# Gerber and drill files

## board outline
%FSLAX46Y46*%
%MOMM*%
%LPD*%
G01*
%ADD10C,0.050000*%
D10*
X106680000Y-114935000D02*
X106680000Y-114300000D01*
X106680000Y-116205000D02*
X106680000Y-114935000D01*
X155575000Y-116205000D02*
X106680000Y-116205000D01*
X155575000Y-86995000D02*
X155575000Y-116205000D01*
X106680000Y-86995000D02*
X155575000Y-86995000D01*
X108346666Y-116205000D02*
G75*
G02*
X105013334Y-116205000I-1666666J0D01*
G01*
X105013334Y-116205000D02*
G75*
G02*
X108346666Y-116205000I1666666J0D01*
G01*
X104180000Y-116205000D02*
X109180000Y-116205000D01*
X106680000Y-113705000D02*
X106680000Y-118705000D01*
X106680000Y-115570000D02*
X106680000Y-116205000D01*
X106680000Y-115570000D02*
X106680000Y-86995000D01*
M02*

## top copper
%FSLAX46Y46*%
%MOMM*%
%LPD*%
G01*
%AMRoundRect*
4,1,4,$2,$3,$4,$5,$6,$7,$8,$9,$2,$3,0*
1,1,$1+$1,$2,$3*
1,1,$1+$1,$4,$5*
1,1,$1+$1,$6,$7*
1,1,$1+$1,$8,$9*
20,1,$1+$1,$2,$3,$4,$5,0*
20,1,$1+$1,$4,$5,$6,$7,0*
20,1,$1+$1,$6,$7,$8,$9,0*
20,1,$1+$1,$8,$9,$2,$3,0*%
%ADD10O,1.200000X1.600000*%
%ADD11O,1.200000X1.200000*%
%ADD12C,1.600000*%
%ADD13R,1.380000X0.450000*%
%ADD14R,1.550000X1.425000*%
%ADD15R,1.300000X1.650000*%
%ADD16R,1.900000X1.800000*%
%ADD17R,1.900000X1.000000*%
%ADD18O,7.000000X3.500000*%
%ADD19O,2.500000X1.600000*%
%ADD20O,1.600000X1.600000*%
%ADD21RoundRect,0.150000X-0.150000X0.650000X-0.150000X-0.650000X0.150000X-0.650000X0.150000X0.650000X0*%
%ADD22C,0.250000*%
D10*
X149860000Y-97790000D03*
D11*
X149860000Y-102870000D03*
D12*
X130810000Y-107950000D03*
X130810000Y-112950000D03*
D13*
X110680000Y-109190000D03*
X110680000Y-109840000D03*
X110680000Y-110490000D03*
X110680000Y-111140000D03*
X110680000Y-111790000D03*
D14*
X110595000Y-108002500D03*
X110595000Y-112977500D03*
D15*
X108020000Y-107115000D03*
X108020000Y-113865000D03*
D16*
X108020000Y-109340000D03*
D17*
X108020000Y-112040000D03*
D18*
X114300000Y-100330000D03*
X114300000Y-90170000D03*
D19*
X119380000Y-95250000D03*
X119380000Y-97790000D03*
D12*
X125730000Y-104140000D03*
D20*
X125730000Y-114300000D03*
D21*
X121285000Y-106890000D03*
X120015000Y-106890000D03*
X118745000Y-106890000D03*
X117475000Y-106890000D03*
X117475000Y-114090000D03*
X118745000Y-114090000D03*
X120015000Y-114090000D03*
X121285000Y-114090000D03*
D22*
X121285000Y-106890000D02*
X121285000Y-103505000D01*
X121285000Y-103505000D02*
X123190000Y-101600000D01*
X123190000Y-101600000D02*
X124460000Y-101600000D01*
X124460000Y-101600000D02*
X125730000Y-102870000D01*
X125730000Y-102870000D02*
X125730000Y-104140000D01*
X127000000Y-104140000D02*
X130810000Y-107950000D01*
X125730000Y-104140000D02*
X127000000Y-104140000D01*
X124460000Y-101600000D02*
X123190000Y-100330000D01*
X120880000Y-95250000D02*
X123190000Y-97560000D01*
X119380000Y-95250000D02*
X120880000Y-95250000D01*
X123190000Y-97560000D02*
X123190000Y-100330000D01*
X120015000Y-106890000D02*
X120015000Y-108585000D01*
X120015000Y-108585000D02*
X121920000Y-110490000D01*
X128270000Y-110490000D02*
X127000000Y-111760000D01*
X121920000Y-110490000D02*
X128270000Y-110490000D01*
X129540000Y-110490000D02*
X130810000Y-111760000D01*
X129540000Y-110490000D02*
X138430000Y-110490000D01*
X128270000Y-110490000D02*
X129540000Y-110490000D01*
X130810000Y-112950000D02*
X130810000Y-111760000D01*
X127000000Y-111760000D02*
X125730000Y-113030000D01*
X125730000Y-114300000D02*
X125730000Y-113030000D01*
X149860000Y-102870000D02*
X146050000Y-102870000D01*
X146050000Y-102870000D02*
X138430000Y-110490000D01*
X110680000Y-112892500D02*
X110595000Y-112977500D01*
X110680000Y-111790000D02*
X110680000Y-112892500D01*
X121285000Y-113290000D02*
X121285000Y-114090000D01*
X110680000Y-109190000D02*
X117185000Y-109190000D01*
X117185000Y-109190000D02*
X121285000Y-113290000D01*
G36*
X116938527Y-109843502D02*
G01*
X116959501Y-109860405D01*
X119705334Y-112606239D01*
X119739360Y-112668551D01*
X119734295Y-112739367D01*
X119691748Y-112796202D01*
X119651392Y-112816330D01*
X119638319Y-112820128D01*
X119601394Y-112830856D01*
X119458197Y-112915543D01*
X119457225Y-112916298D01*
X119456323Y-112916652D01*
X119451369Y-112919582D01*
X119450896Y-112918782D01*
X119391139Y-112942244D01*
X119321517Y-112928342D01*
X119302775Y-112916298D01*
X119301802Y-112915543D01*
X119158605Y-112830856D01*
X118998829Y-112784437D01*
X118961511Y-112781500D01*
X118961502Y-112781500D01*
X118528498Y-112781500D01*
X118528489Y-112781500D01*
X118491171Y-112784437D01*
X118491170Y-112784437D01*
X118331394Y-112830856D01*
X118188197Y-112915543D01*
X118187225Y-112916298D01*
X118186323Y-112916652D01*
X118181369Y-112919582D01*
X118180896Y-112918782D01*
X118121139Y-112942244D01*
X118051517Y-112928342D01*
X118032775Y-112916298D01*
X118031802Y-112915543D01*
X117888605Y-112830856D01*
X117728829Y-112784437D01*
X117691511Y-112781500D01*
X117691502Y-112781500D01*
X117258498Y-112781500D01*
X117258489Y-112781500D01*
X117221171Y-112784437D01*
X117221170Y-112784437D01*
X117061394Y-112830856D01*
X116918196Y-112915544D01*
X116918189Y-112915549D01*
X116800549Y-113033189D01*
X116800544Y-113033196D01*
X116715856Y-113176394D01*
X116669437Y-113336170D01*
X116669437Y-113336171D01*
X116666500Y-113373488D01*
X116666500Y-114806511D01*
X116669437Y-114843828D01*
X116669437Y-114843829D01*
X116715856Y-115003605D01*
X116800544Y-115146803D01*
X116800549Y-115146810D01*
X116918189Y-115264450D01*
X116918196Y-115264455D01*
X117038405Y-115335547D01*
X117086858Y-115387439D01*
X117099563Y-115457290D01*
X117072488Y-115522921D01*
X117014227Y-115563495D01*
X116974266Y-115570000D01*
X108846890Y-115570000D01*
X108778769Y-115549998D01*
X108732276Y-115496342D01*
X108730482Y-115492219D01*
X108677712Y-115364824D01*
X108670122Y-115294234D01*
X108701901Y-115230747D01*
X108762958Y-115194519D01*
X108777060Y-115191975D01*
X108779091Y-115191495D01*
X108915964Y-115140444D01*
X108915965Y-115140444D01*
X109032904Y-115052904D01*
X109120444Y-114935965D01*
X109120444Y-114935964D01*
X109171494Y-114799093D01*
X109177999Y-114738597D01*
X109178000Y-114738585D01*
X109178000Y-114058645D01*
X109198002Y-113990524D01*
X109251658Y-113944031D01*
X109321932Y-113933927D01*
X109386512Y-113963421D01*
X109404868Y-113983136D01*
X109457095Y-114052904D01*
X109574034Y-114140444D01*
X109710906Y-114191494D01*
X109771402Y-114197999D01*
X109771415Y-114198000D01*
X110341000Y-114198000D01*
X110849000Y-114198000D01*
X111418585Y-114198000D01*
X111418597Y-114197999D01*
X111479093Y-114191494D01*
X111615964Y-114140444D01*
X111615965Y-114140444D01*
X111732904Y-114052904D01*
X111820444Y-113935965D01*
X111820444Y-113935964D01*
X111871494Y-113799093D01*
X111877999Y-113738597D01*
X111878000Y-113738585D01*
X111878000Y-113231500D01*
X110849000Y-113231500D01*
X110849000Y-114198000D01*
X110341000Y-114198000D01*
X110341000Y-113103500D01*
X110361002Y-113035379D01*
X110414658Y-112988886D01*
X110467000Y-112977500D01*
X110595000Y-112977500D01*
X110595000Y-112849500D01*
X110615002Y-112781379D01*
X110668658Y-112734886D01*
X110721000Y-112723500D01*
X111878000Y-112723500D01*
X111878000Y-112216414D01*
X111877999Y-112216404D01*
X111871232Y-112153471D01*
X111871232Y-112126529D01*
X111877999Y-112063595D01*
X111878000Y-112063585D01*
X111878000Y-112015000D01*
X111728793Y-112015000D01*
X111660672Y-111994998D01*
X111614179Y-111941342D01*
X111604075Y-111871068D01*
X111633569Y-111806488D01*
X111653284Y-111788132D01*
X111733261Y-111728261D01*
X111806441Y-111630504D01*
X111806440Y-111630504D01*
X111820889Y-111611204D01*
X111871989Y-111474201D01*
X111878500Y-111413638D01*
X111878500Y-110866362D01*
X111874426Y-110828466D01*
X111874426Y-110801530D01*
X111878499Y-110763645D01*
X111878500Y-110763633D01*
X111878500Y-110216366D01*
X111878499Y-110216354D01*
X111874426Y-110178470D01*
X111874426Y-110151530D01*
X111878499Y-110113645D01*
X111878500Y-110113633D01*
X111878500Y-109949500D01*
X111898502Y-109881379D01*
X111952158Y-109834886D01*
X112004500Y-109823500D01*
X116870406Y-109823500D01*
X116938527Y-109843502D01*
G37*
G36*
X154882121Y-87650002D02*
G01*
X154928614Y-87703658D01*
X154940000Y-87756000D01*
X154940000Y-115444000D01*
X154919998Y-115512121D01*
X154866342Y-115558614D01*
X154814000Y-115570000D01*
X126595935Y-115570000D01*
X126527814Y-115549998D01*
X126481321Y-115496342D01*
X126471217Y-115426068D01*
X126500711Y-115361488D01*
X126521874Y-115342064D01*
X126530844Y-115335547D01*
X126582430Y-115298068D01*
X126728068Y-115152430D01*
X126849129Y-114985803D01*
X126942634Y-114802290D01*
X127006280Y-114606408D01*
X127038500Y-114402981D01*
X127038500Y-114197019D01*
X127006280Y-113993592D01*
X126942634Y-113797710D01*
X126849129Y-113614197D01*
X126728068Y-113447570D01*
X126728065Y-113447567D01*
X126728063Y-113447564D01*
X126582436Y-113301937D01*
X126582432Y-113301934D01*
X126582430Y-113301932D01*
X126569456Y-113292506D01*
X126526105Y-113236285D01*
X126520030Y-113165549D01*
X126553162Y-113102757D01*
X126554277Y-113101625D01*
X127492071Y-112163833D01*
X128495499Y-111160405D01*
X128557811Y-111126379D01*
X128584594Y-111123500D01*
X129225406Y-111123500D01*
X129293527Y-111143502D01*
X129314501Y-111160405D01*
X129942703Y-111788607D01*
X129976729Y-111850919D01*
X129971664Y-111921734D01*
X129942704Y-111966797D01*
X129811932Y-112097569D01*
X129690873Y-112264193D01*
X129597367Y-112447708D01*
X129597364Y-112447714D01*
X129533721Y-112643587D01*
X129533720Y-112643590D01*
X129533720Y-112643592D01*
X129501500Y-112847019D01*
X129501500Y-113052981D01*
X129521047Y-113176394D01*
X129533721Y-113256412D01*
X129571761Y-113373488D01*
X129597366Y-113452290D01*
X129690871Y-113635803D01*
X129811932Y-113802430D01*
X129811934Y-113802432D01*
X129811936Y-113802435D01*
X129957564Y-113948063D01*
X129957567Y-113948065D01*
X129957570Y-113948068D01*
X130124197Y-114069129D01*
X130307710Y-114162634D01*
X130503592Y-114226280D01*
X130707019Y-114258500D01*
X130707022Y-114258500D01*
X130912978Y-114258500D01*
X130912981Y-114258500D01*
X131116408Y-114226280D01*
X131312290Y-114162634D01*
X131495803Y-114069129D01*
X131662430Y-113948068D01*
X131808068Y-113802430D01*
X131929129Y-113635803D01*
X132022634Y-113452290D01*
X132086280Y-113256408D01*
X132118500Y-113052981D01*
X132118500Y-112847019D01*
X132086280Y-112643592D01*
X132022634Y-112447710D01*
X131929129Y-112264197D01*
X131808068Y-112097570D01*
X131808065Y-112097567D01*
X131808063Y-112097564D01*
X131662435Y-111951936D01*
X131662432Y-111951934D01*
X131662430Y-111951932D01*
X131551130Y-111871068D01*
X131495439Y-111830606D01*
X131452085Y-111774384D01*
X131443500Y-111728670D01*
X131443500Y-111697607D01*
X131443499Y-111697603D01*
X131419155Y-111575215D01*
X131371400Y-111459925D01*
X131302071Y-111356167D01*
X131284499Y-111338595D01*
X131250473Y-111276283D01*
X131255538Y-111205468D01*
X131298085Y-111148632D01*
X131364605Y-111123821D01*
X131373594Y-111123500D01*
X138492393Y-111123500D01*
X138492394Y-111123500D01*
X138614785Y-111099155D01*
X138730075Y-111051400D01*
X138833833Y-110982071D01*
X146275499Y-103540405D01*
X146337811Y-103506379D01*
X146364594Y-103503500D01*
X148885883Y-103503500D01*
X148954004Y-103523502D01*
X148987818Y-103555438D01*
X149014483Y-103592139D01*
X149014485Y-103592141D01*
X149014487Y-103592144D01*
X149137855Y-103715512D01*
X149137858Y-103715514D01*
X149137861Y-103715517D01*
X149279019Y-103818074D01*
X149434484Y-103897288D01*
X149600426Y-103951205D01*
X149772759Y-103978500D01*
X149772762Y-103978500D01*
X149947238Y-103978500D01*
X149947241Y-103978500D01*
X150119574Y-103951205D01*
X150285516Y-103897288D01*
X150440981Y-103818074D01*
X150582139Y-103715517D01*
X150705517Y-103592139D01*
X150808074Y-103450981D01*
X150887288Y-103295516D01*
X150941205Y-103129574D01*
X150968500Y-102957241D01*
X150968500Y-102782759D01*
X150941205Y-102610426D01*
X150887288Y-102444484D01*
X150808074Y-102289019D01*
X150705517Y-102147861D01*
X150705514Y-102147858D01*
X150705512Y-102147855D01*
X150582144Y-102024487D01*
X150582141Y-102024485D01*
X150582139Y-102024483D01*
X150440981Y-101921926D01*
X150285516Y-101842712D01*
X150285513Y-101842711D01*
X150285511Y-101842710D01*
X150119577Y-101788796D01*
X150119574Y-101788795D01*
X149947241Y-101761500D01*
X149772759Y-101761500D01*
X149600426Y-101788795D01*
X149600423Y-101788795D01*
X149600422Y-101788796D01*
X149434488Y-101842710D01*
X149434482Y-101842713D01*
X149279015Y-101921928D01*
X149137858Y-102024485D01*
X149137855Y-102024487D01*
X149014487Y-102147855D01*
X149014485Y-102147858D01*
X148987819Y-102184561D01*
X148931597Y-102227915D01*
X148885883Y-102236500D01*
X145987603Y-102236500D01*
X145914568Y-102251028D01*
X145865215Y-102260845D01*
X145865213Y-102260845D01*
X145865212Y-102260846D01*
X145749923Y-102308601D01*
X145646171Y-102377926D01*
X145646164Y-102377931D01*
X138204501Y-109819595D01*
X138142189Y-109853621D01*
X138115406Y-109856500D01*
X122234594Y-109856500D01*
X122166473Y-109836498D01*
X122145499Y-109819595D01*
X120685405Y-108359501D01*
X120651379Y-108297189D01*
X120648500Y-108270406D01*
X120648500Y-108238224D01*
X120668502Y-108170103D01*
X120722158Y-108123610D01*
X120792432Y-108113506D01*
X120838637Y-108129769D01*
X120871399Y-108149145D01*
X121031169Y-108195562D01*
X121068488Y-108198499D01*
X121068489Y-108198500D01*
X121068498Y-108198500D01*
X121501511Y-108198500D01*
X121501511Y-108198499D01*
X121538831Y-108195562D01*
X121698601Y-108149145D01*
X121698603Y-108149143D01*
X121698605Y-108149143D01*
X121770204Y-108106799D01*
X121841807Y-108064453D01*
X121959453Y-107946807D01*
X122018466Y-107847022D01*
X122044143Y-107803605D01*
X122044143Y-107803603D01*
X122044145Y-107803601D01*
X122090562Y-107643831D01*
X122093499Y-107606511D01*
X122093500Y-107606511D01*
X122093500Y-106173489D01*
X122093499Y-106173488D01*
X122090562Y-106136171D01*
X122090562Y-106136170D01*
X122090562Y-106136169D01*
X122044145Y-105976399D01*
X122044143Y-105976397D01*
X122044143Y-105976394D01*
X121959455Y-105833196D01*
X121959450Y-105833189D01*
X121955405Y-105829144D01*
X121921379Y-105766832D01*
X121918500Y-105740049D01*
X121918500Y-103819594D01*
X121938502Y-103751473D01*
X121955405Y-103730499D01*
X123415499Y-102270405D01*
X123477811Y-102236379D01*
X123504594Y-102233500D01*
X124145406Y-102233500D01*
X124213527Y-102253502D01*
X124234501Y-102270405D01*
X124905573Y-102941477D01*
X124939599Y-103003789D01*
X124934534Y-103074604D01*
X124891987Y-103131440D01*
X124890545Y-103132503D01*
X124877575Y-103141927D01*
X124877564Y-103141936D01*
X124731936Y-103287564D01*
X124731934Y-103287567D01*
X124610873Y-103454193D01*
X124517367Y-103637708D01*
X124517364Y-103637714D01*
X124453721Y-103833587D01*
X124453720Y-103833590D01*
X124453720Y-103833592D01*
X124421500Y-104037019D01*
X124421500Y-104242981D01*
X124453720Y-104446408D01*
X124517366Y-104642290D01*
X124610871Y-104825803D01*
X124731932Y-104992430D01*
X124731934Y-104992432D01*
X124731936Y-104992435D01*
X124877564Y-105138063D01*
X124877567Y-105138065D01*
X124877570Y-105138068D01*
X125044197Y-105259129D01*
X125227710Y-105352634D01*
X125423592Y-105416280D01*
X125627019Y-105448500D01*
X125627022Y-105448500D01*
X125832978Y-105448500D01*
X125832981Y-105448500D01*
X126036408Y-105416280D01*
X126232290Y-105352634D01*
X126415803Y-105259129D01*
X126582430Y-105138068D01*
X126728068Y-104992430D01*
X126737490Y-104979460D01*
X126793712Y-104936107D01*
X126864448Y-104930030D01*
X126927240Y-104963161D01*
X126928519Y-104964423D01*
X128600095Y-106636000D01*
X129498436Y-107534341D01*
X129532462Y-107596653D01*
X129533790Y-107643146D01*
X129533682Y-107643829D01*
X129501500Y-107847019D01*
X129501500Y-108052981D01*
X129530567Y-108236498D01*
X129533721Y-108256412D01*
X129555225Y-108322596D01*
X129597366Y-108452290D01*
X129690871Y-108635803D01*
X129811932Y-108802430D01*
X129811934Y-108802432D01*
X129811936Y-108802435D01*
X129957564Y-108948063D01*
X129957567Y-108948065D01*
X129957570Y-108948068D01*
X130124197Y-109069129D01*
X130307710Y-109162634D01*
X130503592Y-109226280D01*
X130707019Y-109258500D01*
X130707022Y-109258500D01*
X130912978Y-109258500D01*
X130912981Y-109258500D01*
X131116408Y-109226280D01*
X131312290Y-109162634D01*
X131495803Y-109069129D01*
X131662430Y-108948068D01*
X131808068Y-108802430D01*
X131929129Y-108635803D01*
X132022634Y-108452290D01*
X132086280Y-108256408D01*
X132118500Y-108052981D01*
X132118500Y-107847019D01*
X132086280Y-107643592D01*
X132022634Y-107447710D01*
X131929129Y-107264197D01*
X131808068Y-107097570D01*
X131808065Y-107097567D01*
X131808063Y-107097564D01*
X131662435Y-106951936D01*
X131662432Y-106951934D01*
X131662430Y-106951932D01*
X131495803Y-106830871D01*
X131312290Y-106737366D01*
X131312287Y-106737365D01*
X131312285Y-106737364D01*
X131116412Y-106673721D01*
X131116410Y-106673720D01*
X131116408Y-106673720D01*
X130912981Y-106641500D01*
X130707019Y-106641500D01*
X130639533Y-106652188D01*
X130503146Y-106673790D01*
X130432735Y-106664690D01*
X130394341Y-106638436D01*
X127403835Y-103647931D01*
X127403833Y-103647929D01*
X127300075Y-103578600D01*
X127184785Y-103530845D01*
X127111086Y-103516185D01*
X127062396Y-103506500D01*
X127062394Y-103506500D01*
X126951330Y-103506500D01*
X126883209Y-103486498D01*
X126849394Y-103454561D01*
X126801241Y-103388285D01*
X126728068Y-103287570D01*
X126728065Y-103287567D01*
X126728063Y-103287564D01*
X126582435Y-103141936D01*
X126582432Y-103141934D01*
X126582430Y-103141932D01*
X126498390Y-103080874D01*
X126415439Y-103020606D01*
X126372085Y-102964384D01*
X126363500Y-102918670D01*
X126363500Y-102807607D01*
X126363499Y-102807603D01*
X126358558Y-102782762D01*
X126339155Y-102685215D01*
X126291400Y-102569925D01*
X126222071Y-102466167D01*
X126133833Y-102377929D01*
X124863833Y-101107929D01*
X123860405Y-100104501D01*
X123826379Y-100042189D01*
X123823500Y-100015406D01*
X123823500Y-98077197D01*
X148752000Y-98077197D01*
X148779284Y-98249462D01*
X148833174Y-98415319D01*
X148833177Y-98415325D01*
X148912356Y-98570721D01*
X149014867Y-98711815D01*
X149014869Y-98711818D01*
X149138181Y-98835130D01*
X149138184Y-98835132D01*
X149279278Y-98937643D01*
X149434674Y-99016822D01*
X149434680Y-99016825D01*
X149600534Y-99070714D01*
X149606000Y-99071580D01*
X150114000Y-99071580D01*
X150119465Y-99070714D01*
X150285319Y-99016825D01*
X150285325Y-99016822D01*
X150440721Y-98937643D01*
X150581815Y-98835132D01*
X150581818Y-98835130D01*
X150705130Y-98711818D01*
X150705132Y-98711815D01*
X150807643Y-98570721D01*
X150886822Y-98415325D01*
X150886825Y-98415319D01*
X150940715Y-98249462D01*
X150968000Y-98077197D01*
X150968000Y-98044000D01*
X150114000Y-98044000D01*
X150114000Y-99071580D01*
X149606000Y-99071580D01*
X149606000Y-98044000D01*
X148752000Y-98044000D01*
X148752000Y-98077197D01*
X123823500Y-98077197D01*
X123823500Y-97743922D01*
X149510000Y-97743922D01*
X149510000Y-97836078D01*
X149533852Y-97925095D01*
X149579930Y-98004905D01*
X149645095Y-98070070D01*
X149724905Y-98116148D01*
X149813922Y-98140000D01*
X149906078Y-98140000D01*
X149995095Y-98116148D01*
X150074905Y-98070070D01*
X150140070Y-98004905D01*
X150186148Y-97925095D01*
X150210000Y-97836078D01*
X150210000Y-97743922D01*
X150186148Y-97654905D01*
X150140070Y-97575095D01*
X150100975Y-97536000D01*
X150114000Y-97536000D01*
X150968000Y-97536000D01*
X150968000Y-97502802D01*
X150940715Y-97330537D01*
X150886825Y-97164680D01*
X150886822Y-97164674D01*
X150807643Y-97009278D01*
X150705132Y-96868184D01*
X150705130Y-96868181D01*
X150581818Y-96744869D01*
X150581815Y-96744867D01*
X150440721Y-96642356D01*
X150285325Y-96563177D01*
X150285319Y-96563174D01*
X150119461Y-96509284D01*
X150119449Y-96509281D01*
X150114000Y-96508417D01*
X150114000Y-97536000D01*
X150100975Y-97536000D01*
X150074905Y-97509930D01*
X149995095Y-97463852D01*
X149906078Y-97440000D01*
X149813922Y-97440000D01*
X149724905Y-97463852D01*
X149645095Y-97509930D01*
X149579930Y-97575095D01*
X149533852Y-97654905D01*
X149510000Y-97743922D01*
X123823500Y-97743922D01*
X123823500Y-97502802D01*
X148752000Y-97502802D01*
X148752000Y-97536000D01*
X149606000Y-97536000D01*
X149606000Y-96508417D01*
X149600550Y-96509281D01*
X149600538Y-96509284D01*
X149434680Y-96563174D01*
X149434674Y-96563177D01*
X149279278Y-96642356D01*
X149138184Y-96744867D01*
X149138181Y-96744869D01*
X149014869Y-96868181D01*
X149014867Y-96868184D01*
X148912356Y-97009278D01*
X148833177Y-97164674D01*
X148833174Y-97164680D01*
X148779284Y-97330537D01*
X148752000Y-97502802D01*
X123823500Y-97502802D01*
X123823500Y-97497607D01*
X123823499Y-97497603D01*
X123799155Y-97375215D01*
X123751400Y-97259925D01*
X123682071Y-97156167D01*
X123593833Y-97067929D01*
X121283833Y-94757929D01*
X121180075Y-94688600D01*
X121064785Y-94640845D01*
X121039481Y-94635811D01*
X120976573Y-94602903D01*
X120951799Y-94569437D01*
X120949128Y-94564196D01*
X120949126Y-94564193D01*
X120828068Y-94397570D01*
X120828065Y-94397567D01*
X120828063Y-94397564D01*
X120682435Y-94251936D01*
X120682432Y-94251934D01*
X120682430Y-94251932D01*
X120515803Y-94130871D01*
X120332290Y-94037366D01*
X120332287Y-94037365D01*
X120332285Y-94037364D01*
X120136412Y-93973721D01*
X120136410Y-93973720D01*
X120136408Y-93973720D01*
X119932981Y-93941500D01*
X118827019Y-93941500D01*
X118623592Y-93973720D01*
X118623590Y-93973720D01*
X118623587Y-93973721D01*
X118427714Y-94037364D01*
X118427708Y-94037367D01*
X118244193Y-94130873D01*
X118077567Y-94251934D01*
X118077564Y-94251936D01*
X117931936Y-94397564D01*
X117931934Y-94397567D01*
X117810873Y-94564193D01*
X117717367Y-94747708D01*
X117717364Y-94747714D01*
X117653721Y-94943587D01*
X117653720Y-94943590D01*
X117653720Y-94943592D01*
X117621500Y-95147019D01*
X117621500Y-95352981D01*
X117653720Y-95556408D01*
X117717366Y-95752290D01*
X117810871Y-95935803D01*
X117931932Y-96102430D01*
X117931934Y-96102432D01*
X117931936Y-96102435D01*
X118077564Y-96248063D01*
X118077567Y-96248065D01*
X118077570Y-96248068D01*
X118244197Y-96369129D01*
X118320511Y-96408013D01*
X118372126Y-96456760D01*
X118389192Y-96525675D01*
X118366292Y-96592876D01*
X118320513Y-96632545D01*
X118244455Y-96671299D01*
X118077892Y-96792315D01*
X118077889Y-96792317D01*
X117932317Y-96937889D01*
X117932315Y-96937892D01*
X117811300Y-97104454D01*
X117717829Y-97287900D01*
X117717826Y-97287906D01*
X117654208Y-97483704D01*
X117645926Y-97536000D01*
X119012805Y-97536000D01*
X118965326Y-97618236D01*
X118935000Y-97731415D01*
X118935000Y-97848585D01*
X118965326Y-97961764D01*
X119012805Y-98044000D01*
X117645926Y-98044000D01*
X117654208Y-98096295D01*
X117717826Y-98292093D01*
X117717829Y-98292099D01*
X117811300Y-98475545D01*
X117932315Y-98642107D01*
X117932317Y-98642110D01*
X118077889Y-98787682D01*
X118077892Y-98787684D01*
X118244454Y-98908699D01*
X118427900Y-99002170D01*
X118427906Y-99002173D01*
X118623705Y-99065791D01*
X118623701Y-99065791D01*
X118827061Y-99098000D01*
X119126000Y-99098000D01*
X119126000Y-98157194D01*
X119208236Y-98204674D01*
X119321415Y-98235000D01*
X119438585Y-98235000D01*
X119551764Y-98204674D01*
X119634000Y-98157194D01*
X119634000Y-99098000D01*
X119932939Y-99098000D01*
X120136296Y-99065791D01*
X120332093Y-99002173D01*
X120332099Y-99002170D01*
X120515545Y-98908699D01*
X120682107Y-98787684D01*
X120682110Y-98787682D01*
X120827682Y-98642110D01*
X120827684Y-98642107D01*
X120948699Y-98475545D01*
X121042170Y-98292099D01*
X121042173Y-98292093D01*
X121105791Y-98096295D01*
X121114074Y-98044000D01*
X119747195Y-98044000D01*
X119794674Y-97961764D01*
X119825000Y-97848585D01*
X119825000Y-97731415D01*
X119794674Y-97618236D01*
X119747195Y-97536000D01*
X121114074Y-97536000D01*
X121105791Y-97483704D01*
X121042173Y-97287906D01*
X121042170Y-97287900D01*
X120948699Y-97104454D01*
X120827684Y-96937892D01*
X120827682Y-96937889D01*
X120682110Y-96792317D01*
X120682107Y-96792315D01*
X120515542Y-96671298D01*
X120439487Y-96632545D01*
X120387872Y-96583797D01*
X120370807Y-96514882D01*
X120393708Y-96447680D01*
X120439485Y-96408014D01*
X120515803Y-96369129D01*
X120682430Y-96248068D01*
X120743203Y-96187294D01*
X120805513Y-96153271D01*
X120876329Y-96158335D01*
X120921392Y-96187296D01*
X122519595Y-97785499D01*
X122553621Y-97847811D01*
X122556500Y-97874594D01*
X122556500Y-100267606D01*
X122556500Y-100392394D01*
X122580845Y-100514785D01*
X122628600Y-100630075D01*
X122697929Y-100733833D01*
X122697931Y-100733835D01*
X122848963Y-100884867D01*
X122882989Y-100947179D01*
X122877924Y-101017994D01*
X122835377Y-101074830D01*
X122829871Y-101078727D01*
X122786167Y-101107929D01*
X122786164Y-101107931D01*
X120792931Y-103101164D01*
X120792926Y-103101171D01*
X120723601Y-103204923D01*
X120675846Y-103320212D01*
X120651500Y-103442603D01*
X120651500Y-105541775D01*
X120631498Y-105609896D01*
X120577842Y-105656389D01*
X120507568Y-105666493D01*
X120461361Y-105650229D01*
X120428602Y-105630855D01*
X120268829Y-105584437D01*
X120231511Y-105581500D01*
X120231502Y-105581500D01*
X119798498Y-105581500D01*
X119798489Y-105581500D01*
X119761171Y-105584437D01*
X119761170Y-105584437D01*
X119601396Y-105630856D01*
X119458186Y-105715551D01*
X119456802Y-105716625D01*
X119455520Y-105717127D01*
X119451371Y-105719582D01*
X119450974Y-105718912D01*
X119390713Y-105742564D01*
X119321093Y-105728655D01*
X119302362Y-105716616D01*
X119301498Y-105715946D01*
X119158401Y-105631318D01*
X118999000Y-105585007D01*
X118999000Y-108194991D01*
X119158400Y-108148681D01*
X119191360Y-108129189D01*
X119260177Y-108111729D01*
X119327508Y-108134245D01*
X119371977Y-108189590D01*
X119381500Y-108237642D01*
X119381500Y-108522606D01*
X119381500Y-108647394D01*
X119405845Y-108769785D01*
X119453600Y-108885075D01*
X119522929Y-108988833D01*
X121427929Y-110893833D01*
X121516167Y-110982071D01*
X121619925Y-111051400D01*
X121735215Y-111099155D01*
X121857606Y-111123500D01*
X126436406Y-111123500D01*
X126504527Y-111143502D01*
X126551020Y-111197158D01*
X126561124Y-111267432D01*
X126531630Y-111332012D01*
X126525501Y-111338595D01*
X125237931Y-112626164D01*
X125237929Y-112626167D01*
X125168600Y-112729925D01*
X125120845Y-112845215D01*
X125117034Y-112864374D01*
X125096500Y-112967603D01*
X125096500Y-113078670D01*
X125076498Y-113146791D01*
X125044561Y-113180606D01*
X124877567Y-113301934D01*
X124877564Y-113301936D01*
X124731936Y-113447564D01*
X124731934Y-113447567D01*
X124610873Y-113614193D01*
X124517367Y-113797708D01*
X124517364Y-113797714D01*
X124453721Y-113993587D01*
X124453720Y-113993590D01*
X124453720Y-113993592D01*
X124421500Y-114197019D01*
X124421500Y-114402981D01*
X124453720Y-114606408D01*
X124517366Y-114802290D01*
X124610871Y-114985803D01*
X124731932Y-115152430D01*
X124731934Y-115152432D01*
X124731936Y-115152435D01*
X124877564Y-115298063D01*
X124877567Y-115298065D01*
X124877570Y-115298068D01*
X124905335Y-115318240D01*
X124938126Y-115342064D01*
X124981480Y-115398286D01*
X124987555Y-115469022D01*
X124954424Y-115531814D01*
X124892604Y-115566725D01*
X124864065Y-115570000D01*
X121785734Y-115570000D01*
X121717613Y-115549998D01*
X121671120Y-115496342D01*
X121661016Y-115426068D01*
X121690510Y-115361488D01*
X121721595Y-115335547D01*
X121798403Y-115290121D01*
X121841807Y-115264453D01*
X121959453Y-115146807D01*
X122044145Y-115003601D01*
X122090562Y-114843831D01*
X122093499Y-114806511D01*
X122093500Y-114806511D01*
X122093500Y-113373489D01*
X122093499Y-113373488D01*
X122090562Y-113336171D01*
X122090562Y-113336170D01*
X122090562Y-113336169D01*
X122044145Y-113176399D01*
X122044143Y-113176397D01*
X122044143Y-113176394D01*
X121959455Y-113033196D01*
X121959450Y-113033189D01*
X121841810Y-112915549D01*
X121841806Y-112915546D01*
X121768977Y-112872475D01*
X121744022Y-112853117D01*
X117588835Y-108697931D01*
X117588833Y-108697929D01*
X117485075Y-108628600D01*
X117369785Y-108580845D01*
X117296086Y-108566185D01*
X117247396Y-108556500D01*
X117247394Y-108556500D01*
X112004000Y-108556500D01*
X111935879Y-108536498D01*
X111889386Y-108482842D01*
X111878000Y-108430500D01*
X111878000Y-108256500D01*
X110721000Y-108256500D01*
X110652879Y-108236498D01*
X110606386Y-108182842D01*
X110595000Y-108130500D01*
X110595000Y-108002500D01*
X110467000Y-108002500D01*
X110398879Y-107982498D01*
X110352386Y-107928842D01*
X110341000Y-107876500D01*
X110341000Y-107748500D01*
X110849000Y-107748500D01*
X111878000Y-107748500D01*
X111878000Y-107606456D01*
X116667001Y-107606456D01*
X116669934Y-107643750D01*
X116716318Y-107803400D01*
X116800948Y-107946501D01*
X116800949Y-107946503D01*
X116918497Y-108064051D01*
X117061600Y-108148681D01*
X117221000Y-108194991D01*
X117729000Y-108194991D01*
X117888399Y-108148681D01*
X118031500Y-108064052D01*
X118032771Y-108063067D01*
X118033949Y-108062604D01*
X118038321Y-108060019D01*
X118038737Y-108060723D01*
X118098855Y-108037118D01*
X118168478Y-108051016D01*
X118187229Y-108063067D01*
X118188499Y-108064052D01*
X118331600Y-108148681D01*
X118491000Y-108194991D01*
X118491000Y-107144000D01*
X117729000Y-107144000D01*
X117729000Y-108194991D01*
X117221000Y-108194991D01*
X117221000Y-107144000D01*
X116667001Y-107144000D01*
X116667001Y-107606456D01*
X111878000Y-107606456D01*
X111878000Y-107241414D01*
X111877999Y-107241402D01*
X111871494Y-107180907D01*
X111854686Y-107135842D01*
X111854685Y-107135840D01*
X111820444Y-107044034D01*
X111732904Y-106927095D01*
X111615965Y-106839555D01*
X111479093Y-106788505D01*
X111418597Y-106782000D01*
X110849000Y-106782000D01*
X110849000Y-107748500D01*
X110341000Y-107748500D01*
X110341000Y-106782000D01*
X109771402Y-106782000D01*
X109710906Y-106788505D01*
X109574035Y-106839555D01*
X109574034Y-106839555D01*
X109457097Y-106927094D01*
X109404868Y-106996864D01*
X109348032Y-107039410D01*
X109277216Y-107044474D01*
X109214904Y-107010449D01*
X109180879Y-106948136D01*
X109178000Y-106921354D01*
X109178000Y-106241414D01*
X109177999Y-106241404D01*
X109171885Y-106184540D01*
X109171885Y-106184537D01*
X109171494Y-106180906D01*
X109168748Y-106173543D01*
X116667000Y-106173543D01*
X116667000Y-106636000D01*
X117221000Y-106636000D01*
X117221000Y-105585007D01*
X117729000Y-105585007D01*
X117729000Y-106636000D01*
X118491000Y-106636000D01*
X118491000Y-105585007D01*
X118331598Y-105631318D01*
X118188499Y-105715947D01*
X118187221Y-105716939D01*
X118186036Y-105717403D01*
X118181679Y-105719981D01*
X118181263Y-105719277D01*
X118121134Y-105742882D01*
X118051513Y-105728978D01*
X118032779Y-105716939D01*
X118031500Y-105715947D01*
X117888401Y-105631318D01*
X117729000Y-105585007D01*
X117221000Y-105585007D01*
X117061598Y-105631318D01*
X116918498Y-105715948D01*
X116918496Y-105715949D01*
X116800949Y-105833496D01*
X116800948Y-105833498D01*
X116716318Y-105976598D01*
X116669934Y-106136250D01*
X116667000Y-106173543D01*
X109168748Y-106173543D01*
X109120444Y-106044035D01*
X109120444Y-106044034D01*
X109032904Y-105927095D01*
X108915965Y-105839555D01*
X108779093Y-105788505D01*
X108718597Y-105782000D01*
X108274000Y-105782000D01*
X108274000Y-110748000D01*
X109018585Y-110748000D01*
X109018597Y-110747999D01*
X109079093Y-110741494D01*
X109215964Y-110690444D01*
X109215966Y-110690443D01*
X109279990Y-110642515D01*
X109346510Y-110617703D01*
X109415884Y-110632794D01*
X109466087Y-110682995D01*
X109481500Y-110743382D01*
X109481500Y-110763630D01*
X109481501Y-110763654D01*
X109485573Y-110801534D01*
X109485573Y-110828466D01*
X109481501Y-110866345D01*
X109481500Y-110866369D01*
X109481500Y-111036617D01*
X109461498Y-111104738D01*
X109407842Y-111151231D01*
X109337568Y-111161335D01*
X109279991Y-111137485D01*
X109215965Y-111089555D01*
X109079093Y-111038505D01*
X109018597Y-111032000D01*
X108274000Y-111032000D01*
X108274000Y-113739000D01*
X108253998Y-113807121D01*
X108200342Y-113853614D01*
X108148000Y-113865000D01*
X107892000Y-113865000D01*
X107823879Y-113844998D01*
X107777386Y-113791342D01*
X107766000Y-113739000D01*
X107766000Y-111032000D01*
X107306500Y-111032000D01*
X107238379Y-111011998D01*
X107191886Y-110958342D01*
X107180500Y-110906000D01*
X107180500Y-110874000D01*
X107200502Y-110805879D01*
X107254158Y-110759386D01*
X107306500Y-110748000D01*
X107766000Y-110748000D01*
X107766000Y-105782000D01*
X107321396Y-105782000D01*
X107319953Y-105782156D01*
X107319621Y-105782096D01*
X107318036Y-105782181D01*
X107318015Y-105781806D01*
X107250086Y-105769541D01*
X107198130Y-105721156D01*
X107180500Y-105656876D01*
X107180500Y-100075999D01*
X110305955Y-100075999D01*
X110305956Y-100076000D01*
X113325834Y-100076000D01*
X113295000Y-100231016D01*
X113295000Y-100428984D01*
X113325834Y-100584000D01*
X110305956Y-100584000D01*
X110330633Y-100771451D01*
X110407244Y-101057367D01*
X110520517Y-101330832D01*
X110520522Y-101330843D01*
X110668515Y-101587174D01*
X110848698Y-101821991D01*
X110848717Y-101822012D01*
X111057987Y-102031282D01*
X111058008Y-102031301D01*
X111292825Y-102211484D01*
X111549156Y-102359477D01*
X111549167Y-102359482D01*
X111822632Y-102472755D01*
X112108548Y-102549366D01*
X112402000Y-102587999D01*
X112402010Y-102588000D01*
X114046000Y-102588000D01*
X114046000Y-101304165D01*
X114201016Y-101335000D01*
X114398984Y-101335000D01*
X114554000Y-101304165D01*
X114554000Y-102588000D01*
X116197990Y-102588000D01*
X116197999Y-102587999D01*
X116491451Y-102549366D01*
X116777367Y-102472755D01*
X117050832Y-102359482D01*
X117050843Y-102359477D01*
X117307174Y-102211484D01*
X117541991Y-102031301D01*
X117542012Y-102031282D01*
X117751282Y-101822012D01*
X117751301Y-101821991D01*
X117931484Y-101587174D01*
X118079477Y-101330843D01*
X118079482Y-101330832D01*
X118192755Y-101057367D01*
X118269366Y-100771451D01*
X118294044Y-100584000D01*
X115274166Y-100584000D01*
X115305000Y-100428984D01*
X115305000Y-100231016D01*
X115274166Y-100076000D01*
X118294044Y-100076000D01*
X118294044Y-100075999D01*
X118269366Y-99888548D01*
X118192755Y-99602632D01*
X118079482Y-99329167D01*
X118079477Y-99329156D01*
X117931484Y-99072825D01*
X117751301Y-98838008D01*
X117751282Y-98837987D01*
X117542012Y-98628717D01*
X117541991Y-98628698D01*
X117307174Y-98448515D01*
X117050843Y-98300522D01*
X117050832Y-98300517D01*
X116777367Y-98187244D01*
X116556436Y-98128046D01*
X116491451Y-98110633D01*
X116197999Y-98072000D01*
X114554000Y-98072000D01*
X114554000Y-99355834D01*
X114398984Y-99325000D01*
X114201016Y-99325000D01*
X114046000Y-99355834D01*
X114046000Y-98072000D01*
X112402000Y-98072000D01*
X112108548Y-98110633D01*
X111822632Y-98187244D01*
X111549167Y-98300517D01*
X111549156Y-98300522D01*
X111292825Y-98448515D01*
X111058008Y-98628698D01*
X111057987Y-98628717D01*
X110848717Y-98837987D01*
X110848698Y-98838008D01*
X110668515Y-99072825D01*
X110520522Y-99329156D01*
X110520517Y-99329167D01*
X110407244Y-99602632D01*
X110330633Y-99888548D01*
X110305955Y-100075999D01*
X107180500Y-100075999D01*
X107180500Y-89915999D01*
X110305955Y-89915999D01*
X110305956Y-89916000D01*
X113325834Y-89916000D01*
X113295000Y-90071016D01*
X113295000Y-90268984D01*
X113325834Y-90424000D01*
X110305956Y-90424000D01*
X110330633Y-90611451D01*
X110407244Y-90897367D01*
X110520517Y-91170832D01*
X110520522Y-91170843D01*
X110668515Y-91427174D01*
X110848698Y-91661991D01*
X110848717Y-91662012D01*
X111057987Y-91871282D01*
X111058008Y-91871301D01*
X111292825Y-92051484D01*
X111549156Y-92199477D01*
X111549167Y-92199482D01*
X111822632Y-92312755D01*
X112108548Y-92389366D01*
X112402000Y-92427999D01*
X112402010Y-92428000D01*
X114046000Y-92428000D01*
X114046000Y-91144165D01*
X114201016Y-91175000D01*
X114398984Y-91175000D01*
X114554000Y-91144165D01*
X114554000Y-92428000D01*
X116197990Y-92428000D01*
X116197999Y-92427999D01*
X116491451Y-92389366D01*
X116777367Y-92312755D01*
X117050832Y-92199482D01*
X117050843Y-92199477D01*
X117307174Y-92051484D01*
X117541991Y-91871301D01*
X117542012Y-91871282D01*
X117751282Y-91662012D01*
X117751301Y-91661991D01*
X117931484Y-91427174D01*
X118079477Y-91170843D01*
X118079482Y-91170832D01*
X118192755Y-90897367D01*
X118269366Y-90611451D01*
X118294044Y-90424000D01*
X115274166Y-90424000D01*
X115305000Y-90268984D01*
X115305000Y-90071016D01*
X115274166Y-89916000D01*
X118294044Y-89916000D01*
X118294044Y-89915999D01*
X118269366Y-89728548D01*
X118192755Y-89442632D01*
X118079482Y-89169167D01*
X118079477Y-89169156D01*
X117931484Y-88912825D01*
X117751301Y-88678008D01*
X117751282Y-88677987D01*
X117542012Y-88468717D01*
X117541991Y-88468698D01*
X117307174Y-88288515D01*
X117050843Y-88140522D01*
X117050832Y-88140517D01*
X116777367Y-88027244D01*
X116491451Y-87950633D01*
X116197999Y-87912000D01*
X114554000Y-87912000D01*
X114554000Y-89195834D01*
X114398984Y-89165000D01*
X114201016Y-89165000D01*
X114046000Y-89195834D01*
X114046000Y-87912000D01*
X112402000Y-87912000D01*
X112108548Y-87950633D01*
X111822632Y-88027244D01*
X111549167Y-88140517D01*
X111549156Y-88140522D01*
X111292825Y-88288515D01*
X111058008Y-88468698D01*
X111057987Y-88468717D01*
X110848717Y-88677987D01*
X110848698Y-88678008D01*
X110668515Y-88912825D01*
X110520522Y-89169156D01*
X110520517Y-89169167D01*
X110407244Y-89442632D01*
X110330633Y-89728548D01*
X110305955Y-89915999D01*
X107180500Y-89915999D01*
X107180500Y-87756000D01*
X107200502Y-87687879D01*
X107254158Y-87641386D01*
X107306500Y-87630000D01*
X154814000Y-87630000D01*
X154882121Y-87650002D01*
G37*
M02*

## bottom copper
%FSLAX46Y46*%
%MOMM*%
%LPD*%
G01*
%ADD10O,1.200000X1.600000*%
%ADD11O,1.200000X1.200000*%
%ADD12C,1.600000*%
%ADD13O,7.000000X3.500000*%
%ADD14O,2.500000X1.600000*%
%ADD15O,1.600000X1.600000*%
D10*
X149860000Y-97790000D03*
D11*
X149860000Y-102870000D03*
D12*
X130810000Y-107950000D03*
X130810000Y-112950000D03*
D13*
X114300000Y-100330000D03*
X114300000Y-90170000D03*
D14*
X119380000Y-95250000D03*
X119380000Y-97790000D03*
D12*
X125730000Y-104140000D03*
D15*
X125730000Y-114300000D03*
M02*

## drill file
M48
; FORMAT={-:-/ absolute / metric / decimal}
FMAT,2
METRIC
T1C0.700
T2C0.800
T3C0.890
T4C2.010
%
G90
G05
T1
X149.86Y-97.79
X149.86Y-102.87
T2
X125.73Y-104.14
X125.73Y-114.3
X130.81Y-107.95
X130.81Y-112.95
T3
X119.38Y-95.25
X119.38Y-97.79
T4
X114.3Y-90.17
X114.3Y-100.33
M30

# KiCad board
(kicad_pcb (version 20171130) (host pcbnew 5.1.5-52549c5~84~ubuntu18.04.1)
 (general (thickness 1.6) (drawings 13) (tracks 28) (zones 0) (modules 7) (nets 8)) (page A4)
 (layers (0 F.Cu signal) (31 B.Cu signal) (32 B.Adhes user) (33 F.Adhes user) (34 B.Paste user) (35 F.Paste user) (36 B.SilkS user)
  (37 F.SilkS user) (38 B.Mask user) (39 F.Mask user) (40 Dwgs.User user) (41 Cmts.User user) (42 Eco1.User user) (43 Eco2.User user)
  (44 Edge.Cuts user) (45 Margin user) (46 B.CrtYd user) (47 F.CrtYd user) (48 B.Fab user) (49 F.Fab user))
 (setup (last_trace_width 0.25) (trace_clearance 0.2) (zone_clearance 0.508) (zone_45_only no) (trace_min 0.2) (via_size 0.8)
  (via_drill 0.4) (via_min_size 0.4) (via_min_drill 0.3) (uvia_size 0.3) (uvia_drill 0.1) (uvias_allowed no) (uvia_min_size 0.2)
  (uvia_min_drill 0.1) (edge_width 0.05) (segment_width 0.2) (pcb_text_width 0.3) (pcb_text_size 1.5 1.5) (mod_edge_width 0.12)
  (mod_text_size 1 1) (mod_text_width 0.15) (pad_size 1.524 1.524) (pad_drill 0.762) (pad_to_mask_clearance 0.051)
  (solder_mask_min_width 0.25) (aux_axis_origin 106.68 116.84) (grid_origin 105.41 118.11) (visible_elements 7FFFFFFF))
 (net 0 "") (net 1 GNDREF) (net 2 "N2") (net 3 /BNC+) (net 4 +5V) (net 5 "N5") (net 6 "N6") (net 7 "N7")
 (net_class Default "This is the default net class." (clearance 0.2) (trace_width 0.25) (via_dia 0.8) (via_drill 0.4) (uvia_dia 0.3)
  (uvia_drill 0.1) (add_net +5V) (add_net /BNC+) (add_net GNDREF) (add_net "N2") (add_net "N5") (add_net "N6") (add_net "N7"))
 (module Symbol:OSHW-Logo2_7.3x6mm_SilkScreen (layer F.Cu) (at 151.13 90.805)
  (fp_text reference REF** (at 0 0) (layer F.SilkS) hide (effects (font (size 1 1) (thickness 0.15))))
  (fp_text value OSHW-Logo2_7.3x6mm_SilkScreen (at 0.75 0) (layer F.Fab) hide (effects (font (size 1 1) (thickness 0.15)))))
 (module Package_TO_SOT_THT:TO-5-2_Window (layer F.Cu) (at 149.86 97.79 270)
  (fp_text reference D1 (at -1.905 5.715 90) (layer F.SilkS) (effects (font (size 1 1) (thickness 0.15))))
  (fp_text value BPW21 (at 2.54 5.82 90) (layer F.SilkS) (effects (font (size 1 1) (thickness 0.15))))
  (pad 1 thru_hole oval (at 0 0 270) (size 1.6 1.2) (drill 0.7) (layers *.Cu *.Mask) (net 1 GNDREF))
  (pad 2 thru_hole oval (at 5.08 0 270) (size 1.2 1.2) (drill 0.7) (layers *.Cu *.Mask) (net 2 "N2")))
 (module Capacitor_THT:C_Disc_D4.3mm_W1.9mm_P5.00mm (layer F.Cu) (at 130.81 107.95 270)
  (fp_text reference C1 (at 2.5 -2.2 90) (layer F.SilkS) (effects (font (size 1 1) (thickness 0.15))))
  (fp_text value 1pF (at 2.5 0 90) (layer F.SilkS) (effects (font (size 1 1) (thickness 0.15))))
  (pad 1 thru_hole circle (at 0 0 270) (size 1.6 1.6) (drill 0.8) (layers *.Cu *.Mask) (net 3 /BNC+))
  (pad 2 thru_hole circle (at 5 0 270) (size 1.6 1.6) (drill 0.8) (layers *.Cu *.Mask) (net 2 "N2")))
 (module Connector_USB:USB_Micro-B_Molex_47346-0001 (layer F.Cu) (at 109.22 110.49 270)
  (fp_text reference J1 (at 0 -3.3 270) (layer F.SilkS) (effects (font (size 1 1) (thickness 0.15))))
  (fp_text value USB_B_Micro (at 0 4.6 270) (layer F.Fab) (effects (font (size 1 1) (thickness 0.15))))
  (pad 1 smd rect (at -1.3 -1.46 270) (size 0.45 1.38) (layers F.Cu F.Paste F.Mask) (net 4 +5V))
  (pad 2 smd rect (at -0.65 -1.46 270) (size 0.45 1.38) (layers F.Cu F.Paste F.Mask) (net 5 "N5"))
  (pad 3 smd rect (at 0 -1.46 270) (size 0.45 1.38) (layers F.Cu F.Paste F.Mask) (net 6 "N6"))
  (pad 4 smd rect (at 0.65 -1.46 270) (size 0.45 1.38) (layers F.Cu F.Paste F.Mask) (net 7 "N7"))
  (pad 5 smd rect (at 1.3 -1.46 270) (size 0.45 1.38) (layers F.Cu F.Paste F.Mask) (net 1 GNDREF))
  (pad 6 smd rect (at -2.4875 -1.375 270) (size 1.425 1.55) (layers F.Cu F.Paste F.Mask) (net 1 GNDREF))
  (pad 6 smd rect (at 2.4875 -1.375 270) (size 1.425 1.55) (layers F.Cu F.Paste F.Mask) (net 1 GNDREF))
  (pad 6 smd rect (at -3.375 1.2 270) (size 1.65 1.3) (layers F.Cu F.Paste F.Mask) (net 1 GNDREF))
  (pad 6 smd rect (at 3.375 1.2 270) (size 1.65 1.3) (layers F.Cu F.Paste F.Mask) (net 1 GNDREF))
  (pad 6 smd rect (at -1.15 1.2 270) (size 1.8 1.9) (layers F.Cu F.Paste F.Mask) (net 1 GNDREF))
  (pad 6 smd rect (at 1.55 1.2 270) (size 1 1.9) (layers F.Cu F.Paste F.Mask) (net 1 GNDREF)))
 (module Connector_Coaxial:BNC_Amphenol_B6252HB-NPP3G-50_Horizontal (layer F.Cu) (at 119.38 95.25 90)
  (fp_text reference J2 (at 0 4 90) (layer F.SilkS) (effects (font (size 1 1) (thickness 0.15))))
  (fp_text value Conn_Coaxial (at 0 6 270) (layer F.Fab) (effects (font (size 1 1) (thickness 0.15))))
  (pad 2 thru_hole oval (at -5.08 -5.08 90) (size 3.5 7) (drill 2.01) (layers *.Cu *.Mask) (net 1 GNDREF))
  (pad 2 thru_hole oval (at 5.08 -5.08 90) (size 3.5 7) (drill 2.01) (layers *.Cu *.Mask) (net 1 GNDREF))
  (pad 1 thru_hole oval (at 0 0 90) (size 1.6 2.5) (drill 0.89) (layers *.Cu *.Mask) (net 3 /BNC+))
  (pad 2 thru_hole oval (at -2.54 0 90) (size 1.6 2.5) (drill 0.89) (layers *.Cu *.Mask) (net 1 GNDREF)))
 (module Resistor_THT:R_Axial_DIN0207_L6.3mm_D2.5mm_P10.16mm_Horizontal (layer F.Cu) (at 125.73 104.14 270)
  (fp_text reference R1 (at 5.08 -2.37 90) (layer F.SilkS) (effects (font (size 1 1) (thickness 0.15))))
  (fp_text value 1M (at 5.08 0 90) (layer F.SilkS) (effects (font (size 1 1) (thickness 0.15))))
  (pad 1 thru_hole circle (at 0 0 270) (size 1.6 1.6) (drill 0.8) (layers *.Cu *.Mask) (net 3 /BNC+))
  (pad 2 thru_hole oval (at 10.16 0 270) (size 1.6 1.6) (drill 0.8) (layers *.Cu *.Mask) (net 2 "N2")))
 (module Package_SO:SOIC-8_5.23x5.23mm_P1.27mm (layer F.Cu) (at 119.38 110.49 270)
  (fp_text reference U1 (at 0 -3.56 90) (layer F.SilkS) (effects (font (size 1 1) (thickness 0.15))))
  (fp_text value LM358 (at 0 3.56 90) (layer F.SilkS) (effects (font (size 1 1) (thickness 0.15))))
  (pad 1 smd roundrect (at -3.6 -1.905 270) (size 1.6 0.6) (layers F.Cu F.Paste F.Mask) (roundrect_rratio 0.25) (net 3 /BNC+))
  (pad 2 smd roundrect (at -3.6 -0.635 270) (size 1.6 0.6) (layers F.Cu F.Paste F.Mask) (roundrect_rratio 0.25) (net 2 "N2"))
  (pad 3 smd roundrect (at -3.6 0.635 270) (size 1.6 0.6) (layers F.Cu F.Paste F.Mask) (roundrect_rratio 0.25) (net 1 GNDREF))
  (pad 4 smd roundrect (at -3.6 1.905 270) (size 1.6 0.6) (layers F.Cu F.Paste F.Mask) (roundrect_rratio 0.25) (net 1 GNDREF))
  (pad 5 smd roundrect (at 3.6 1.905 270) (size 1.6 0.6) (layers F.Cu F.Paste F.Mask) (roundrect_rratio 0.25))
  (pad 6 smd roundrect (at 3.6 0.635 270) (size 1.6 0.6) (layers F.Cu F.Paste F.Mask) (roundrect_rratio 0.25))
  (pad 7 smd roundrect (at 3.6 -0.635 270) (size 1.6 0.6) (layers F.Cu F.Paste F.Mask) (roundrect_rratio 0.25))
  (pad 8 smd roundrect (at 3.6 -1.905 270) (size 1.6 0.6) (layers F.Cu F.Paste F.Mask) (roundrect_rratio 0.25) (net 4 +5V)))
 (gr_line (start 106.68 114.935) (end 106.68 114.3) (layer Edge.Cuts) (width 0.05))
 (gr_line (start 106.68 116.205) (end 106.68 114.935) (layer Edge.Cuts) (width 0.05))
 (gr_line (start 155.575 116.205) (end 106.68 116.205) (layer Edge.Cuts) (width 0.05))
 (gr_line (start 155.575 86.995) (end 155.575 116.205) (layer Edge.Cuts) (width 0.05))
 (gr_line (start 106.68 86.995) (end 155.575 86.995) (layer Edge.Cuts) (width 0.05))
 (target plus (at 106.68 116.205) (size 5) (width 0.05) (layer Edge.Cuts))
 (gr_line (start 106.68 115.57) (end 106.68 116.205) (layer Edge.Cuts) (width 0.05))
 (gr_line (start 106.68 115.57) (end 106.68 86.995) (layer Edge.Cuts) (width 0.05))
 (segment (start 121.285 106.89) (end 121.285 103.505) (width 0.25) (layer F.Cu) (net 3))
 (segment (start 121.285 103.505) (end 123.19 101.6) (width 0.25) (layer F.Cu) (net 3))
 (segment (start 123.19 101.6) (end 124.46 101.6) (width 0.25) (layer F.Cu) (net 3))
 (segment (start 124.46 101.6) (end 125.73 102.87) (width 0.25) (layer F.Cu) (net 3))
 (segment (start 125.73 102.87) (end 125.73 104.14) (width 0.25) (layer F.Cu) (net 3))
 (segment (start 127 104.14) (end 130.81 107.95) (width 0.25) (layer F.Cu) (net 3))
 (segment (start 125.73 104.14) (end 127 104.14) (width 0.25) (layer F.Cu) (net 3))
 (segment (start 124.46 101.6) (end 123.19 100.33) (width 0.25) (layer F.Cu) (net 3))
 (segment (start 120.88 95.25) (end 123.19 97.56) (width 0.25) (layer F.Cu) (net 3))
 (segment (start 119.38 95.25) (end 120.88 95.25) (width 0.25) (layer F.Cu) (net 3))
 (segment (start 123.19 97.56) (end 123.19 100.33) (width 0.25) (layer F.Cu) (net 3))
 (segment (start 120.015 106.89) (end 120.015 108.585) (width 0.25) (layer F.Cu) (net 2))
 (segment (start 120.015 108.585) (end 121.92 110.49) (width 0.25) (layer F.Cu) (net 2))
 (segment (start 128.27 110.49) (end 127 111.76) (width 0.25) (layer F.Cu) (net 2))
 (segment (start 121.92 110.49) (end 128.27 110.49) (width 0.25) (layer F.Cu) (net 2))
 (segment (start 129.54 110.49) (end 130.81 111.76) (width 0.25) (layer F.Cu) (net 2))
 (segment (start 129.54 110.49) (end 138.43 110.49) (width 0.25) (layer F.Cu) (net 2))
 (segment (start 128.27 110.49) (end 129.54 110.49) (width 0.25) (layer F.Cu) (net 2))
 (segment (start 130.81 112.95) (end 130.81 111.76) (width 0.25) (layer F.Cu) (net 2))
 (segment (start 127 111.76) (end 125.73 113.03) (width 0.25) (layer F.Cu) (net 2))
 (segment (start 125.73 114.3) (end 125.73 113.03) (width 0.25) (layer F.Cu) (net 2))
 (segment (start 149.86 102.87) (end 146.05 102.87) (width 0.25) (layer F.Cu) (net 2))
 (segment (start 146.05 102.87) (end 138.43 110.49) (width 0.25) (layer F.Cu) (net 2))
 (segment (start 110.68 112.8925) (end 110.595 112.9775) (width 0.25) (layer F.Cu) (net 1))
 (segment (start 110.68 111.79) (end 110.68 112.8925) (width 0.25) (layer F.Cu) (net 1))
 (segment (start 121.285 113.29) (end 121.285 114.09) (width 0.25) (layer F.Cu) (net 4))
 (segment (start 110.68 109.19) (end 117.185 109.19) (width 0.25) (layer F.Cu) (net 4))
 (segment (start 117.185 109.19) (end 121.285 113.29) (width 0.25) (layer F.Cu) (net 4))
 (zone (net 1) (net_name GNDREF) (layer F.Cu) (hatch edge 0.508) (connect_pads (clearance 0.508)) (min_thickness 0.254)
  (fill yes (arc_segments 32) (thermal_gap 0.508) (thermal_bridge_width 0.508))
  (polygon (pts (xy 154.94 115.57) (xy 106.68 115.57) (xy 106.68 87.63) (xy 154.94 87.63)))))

